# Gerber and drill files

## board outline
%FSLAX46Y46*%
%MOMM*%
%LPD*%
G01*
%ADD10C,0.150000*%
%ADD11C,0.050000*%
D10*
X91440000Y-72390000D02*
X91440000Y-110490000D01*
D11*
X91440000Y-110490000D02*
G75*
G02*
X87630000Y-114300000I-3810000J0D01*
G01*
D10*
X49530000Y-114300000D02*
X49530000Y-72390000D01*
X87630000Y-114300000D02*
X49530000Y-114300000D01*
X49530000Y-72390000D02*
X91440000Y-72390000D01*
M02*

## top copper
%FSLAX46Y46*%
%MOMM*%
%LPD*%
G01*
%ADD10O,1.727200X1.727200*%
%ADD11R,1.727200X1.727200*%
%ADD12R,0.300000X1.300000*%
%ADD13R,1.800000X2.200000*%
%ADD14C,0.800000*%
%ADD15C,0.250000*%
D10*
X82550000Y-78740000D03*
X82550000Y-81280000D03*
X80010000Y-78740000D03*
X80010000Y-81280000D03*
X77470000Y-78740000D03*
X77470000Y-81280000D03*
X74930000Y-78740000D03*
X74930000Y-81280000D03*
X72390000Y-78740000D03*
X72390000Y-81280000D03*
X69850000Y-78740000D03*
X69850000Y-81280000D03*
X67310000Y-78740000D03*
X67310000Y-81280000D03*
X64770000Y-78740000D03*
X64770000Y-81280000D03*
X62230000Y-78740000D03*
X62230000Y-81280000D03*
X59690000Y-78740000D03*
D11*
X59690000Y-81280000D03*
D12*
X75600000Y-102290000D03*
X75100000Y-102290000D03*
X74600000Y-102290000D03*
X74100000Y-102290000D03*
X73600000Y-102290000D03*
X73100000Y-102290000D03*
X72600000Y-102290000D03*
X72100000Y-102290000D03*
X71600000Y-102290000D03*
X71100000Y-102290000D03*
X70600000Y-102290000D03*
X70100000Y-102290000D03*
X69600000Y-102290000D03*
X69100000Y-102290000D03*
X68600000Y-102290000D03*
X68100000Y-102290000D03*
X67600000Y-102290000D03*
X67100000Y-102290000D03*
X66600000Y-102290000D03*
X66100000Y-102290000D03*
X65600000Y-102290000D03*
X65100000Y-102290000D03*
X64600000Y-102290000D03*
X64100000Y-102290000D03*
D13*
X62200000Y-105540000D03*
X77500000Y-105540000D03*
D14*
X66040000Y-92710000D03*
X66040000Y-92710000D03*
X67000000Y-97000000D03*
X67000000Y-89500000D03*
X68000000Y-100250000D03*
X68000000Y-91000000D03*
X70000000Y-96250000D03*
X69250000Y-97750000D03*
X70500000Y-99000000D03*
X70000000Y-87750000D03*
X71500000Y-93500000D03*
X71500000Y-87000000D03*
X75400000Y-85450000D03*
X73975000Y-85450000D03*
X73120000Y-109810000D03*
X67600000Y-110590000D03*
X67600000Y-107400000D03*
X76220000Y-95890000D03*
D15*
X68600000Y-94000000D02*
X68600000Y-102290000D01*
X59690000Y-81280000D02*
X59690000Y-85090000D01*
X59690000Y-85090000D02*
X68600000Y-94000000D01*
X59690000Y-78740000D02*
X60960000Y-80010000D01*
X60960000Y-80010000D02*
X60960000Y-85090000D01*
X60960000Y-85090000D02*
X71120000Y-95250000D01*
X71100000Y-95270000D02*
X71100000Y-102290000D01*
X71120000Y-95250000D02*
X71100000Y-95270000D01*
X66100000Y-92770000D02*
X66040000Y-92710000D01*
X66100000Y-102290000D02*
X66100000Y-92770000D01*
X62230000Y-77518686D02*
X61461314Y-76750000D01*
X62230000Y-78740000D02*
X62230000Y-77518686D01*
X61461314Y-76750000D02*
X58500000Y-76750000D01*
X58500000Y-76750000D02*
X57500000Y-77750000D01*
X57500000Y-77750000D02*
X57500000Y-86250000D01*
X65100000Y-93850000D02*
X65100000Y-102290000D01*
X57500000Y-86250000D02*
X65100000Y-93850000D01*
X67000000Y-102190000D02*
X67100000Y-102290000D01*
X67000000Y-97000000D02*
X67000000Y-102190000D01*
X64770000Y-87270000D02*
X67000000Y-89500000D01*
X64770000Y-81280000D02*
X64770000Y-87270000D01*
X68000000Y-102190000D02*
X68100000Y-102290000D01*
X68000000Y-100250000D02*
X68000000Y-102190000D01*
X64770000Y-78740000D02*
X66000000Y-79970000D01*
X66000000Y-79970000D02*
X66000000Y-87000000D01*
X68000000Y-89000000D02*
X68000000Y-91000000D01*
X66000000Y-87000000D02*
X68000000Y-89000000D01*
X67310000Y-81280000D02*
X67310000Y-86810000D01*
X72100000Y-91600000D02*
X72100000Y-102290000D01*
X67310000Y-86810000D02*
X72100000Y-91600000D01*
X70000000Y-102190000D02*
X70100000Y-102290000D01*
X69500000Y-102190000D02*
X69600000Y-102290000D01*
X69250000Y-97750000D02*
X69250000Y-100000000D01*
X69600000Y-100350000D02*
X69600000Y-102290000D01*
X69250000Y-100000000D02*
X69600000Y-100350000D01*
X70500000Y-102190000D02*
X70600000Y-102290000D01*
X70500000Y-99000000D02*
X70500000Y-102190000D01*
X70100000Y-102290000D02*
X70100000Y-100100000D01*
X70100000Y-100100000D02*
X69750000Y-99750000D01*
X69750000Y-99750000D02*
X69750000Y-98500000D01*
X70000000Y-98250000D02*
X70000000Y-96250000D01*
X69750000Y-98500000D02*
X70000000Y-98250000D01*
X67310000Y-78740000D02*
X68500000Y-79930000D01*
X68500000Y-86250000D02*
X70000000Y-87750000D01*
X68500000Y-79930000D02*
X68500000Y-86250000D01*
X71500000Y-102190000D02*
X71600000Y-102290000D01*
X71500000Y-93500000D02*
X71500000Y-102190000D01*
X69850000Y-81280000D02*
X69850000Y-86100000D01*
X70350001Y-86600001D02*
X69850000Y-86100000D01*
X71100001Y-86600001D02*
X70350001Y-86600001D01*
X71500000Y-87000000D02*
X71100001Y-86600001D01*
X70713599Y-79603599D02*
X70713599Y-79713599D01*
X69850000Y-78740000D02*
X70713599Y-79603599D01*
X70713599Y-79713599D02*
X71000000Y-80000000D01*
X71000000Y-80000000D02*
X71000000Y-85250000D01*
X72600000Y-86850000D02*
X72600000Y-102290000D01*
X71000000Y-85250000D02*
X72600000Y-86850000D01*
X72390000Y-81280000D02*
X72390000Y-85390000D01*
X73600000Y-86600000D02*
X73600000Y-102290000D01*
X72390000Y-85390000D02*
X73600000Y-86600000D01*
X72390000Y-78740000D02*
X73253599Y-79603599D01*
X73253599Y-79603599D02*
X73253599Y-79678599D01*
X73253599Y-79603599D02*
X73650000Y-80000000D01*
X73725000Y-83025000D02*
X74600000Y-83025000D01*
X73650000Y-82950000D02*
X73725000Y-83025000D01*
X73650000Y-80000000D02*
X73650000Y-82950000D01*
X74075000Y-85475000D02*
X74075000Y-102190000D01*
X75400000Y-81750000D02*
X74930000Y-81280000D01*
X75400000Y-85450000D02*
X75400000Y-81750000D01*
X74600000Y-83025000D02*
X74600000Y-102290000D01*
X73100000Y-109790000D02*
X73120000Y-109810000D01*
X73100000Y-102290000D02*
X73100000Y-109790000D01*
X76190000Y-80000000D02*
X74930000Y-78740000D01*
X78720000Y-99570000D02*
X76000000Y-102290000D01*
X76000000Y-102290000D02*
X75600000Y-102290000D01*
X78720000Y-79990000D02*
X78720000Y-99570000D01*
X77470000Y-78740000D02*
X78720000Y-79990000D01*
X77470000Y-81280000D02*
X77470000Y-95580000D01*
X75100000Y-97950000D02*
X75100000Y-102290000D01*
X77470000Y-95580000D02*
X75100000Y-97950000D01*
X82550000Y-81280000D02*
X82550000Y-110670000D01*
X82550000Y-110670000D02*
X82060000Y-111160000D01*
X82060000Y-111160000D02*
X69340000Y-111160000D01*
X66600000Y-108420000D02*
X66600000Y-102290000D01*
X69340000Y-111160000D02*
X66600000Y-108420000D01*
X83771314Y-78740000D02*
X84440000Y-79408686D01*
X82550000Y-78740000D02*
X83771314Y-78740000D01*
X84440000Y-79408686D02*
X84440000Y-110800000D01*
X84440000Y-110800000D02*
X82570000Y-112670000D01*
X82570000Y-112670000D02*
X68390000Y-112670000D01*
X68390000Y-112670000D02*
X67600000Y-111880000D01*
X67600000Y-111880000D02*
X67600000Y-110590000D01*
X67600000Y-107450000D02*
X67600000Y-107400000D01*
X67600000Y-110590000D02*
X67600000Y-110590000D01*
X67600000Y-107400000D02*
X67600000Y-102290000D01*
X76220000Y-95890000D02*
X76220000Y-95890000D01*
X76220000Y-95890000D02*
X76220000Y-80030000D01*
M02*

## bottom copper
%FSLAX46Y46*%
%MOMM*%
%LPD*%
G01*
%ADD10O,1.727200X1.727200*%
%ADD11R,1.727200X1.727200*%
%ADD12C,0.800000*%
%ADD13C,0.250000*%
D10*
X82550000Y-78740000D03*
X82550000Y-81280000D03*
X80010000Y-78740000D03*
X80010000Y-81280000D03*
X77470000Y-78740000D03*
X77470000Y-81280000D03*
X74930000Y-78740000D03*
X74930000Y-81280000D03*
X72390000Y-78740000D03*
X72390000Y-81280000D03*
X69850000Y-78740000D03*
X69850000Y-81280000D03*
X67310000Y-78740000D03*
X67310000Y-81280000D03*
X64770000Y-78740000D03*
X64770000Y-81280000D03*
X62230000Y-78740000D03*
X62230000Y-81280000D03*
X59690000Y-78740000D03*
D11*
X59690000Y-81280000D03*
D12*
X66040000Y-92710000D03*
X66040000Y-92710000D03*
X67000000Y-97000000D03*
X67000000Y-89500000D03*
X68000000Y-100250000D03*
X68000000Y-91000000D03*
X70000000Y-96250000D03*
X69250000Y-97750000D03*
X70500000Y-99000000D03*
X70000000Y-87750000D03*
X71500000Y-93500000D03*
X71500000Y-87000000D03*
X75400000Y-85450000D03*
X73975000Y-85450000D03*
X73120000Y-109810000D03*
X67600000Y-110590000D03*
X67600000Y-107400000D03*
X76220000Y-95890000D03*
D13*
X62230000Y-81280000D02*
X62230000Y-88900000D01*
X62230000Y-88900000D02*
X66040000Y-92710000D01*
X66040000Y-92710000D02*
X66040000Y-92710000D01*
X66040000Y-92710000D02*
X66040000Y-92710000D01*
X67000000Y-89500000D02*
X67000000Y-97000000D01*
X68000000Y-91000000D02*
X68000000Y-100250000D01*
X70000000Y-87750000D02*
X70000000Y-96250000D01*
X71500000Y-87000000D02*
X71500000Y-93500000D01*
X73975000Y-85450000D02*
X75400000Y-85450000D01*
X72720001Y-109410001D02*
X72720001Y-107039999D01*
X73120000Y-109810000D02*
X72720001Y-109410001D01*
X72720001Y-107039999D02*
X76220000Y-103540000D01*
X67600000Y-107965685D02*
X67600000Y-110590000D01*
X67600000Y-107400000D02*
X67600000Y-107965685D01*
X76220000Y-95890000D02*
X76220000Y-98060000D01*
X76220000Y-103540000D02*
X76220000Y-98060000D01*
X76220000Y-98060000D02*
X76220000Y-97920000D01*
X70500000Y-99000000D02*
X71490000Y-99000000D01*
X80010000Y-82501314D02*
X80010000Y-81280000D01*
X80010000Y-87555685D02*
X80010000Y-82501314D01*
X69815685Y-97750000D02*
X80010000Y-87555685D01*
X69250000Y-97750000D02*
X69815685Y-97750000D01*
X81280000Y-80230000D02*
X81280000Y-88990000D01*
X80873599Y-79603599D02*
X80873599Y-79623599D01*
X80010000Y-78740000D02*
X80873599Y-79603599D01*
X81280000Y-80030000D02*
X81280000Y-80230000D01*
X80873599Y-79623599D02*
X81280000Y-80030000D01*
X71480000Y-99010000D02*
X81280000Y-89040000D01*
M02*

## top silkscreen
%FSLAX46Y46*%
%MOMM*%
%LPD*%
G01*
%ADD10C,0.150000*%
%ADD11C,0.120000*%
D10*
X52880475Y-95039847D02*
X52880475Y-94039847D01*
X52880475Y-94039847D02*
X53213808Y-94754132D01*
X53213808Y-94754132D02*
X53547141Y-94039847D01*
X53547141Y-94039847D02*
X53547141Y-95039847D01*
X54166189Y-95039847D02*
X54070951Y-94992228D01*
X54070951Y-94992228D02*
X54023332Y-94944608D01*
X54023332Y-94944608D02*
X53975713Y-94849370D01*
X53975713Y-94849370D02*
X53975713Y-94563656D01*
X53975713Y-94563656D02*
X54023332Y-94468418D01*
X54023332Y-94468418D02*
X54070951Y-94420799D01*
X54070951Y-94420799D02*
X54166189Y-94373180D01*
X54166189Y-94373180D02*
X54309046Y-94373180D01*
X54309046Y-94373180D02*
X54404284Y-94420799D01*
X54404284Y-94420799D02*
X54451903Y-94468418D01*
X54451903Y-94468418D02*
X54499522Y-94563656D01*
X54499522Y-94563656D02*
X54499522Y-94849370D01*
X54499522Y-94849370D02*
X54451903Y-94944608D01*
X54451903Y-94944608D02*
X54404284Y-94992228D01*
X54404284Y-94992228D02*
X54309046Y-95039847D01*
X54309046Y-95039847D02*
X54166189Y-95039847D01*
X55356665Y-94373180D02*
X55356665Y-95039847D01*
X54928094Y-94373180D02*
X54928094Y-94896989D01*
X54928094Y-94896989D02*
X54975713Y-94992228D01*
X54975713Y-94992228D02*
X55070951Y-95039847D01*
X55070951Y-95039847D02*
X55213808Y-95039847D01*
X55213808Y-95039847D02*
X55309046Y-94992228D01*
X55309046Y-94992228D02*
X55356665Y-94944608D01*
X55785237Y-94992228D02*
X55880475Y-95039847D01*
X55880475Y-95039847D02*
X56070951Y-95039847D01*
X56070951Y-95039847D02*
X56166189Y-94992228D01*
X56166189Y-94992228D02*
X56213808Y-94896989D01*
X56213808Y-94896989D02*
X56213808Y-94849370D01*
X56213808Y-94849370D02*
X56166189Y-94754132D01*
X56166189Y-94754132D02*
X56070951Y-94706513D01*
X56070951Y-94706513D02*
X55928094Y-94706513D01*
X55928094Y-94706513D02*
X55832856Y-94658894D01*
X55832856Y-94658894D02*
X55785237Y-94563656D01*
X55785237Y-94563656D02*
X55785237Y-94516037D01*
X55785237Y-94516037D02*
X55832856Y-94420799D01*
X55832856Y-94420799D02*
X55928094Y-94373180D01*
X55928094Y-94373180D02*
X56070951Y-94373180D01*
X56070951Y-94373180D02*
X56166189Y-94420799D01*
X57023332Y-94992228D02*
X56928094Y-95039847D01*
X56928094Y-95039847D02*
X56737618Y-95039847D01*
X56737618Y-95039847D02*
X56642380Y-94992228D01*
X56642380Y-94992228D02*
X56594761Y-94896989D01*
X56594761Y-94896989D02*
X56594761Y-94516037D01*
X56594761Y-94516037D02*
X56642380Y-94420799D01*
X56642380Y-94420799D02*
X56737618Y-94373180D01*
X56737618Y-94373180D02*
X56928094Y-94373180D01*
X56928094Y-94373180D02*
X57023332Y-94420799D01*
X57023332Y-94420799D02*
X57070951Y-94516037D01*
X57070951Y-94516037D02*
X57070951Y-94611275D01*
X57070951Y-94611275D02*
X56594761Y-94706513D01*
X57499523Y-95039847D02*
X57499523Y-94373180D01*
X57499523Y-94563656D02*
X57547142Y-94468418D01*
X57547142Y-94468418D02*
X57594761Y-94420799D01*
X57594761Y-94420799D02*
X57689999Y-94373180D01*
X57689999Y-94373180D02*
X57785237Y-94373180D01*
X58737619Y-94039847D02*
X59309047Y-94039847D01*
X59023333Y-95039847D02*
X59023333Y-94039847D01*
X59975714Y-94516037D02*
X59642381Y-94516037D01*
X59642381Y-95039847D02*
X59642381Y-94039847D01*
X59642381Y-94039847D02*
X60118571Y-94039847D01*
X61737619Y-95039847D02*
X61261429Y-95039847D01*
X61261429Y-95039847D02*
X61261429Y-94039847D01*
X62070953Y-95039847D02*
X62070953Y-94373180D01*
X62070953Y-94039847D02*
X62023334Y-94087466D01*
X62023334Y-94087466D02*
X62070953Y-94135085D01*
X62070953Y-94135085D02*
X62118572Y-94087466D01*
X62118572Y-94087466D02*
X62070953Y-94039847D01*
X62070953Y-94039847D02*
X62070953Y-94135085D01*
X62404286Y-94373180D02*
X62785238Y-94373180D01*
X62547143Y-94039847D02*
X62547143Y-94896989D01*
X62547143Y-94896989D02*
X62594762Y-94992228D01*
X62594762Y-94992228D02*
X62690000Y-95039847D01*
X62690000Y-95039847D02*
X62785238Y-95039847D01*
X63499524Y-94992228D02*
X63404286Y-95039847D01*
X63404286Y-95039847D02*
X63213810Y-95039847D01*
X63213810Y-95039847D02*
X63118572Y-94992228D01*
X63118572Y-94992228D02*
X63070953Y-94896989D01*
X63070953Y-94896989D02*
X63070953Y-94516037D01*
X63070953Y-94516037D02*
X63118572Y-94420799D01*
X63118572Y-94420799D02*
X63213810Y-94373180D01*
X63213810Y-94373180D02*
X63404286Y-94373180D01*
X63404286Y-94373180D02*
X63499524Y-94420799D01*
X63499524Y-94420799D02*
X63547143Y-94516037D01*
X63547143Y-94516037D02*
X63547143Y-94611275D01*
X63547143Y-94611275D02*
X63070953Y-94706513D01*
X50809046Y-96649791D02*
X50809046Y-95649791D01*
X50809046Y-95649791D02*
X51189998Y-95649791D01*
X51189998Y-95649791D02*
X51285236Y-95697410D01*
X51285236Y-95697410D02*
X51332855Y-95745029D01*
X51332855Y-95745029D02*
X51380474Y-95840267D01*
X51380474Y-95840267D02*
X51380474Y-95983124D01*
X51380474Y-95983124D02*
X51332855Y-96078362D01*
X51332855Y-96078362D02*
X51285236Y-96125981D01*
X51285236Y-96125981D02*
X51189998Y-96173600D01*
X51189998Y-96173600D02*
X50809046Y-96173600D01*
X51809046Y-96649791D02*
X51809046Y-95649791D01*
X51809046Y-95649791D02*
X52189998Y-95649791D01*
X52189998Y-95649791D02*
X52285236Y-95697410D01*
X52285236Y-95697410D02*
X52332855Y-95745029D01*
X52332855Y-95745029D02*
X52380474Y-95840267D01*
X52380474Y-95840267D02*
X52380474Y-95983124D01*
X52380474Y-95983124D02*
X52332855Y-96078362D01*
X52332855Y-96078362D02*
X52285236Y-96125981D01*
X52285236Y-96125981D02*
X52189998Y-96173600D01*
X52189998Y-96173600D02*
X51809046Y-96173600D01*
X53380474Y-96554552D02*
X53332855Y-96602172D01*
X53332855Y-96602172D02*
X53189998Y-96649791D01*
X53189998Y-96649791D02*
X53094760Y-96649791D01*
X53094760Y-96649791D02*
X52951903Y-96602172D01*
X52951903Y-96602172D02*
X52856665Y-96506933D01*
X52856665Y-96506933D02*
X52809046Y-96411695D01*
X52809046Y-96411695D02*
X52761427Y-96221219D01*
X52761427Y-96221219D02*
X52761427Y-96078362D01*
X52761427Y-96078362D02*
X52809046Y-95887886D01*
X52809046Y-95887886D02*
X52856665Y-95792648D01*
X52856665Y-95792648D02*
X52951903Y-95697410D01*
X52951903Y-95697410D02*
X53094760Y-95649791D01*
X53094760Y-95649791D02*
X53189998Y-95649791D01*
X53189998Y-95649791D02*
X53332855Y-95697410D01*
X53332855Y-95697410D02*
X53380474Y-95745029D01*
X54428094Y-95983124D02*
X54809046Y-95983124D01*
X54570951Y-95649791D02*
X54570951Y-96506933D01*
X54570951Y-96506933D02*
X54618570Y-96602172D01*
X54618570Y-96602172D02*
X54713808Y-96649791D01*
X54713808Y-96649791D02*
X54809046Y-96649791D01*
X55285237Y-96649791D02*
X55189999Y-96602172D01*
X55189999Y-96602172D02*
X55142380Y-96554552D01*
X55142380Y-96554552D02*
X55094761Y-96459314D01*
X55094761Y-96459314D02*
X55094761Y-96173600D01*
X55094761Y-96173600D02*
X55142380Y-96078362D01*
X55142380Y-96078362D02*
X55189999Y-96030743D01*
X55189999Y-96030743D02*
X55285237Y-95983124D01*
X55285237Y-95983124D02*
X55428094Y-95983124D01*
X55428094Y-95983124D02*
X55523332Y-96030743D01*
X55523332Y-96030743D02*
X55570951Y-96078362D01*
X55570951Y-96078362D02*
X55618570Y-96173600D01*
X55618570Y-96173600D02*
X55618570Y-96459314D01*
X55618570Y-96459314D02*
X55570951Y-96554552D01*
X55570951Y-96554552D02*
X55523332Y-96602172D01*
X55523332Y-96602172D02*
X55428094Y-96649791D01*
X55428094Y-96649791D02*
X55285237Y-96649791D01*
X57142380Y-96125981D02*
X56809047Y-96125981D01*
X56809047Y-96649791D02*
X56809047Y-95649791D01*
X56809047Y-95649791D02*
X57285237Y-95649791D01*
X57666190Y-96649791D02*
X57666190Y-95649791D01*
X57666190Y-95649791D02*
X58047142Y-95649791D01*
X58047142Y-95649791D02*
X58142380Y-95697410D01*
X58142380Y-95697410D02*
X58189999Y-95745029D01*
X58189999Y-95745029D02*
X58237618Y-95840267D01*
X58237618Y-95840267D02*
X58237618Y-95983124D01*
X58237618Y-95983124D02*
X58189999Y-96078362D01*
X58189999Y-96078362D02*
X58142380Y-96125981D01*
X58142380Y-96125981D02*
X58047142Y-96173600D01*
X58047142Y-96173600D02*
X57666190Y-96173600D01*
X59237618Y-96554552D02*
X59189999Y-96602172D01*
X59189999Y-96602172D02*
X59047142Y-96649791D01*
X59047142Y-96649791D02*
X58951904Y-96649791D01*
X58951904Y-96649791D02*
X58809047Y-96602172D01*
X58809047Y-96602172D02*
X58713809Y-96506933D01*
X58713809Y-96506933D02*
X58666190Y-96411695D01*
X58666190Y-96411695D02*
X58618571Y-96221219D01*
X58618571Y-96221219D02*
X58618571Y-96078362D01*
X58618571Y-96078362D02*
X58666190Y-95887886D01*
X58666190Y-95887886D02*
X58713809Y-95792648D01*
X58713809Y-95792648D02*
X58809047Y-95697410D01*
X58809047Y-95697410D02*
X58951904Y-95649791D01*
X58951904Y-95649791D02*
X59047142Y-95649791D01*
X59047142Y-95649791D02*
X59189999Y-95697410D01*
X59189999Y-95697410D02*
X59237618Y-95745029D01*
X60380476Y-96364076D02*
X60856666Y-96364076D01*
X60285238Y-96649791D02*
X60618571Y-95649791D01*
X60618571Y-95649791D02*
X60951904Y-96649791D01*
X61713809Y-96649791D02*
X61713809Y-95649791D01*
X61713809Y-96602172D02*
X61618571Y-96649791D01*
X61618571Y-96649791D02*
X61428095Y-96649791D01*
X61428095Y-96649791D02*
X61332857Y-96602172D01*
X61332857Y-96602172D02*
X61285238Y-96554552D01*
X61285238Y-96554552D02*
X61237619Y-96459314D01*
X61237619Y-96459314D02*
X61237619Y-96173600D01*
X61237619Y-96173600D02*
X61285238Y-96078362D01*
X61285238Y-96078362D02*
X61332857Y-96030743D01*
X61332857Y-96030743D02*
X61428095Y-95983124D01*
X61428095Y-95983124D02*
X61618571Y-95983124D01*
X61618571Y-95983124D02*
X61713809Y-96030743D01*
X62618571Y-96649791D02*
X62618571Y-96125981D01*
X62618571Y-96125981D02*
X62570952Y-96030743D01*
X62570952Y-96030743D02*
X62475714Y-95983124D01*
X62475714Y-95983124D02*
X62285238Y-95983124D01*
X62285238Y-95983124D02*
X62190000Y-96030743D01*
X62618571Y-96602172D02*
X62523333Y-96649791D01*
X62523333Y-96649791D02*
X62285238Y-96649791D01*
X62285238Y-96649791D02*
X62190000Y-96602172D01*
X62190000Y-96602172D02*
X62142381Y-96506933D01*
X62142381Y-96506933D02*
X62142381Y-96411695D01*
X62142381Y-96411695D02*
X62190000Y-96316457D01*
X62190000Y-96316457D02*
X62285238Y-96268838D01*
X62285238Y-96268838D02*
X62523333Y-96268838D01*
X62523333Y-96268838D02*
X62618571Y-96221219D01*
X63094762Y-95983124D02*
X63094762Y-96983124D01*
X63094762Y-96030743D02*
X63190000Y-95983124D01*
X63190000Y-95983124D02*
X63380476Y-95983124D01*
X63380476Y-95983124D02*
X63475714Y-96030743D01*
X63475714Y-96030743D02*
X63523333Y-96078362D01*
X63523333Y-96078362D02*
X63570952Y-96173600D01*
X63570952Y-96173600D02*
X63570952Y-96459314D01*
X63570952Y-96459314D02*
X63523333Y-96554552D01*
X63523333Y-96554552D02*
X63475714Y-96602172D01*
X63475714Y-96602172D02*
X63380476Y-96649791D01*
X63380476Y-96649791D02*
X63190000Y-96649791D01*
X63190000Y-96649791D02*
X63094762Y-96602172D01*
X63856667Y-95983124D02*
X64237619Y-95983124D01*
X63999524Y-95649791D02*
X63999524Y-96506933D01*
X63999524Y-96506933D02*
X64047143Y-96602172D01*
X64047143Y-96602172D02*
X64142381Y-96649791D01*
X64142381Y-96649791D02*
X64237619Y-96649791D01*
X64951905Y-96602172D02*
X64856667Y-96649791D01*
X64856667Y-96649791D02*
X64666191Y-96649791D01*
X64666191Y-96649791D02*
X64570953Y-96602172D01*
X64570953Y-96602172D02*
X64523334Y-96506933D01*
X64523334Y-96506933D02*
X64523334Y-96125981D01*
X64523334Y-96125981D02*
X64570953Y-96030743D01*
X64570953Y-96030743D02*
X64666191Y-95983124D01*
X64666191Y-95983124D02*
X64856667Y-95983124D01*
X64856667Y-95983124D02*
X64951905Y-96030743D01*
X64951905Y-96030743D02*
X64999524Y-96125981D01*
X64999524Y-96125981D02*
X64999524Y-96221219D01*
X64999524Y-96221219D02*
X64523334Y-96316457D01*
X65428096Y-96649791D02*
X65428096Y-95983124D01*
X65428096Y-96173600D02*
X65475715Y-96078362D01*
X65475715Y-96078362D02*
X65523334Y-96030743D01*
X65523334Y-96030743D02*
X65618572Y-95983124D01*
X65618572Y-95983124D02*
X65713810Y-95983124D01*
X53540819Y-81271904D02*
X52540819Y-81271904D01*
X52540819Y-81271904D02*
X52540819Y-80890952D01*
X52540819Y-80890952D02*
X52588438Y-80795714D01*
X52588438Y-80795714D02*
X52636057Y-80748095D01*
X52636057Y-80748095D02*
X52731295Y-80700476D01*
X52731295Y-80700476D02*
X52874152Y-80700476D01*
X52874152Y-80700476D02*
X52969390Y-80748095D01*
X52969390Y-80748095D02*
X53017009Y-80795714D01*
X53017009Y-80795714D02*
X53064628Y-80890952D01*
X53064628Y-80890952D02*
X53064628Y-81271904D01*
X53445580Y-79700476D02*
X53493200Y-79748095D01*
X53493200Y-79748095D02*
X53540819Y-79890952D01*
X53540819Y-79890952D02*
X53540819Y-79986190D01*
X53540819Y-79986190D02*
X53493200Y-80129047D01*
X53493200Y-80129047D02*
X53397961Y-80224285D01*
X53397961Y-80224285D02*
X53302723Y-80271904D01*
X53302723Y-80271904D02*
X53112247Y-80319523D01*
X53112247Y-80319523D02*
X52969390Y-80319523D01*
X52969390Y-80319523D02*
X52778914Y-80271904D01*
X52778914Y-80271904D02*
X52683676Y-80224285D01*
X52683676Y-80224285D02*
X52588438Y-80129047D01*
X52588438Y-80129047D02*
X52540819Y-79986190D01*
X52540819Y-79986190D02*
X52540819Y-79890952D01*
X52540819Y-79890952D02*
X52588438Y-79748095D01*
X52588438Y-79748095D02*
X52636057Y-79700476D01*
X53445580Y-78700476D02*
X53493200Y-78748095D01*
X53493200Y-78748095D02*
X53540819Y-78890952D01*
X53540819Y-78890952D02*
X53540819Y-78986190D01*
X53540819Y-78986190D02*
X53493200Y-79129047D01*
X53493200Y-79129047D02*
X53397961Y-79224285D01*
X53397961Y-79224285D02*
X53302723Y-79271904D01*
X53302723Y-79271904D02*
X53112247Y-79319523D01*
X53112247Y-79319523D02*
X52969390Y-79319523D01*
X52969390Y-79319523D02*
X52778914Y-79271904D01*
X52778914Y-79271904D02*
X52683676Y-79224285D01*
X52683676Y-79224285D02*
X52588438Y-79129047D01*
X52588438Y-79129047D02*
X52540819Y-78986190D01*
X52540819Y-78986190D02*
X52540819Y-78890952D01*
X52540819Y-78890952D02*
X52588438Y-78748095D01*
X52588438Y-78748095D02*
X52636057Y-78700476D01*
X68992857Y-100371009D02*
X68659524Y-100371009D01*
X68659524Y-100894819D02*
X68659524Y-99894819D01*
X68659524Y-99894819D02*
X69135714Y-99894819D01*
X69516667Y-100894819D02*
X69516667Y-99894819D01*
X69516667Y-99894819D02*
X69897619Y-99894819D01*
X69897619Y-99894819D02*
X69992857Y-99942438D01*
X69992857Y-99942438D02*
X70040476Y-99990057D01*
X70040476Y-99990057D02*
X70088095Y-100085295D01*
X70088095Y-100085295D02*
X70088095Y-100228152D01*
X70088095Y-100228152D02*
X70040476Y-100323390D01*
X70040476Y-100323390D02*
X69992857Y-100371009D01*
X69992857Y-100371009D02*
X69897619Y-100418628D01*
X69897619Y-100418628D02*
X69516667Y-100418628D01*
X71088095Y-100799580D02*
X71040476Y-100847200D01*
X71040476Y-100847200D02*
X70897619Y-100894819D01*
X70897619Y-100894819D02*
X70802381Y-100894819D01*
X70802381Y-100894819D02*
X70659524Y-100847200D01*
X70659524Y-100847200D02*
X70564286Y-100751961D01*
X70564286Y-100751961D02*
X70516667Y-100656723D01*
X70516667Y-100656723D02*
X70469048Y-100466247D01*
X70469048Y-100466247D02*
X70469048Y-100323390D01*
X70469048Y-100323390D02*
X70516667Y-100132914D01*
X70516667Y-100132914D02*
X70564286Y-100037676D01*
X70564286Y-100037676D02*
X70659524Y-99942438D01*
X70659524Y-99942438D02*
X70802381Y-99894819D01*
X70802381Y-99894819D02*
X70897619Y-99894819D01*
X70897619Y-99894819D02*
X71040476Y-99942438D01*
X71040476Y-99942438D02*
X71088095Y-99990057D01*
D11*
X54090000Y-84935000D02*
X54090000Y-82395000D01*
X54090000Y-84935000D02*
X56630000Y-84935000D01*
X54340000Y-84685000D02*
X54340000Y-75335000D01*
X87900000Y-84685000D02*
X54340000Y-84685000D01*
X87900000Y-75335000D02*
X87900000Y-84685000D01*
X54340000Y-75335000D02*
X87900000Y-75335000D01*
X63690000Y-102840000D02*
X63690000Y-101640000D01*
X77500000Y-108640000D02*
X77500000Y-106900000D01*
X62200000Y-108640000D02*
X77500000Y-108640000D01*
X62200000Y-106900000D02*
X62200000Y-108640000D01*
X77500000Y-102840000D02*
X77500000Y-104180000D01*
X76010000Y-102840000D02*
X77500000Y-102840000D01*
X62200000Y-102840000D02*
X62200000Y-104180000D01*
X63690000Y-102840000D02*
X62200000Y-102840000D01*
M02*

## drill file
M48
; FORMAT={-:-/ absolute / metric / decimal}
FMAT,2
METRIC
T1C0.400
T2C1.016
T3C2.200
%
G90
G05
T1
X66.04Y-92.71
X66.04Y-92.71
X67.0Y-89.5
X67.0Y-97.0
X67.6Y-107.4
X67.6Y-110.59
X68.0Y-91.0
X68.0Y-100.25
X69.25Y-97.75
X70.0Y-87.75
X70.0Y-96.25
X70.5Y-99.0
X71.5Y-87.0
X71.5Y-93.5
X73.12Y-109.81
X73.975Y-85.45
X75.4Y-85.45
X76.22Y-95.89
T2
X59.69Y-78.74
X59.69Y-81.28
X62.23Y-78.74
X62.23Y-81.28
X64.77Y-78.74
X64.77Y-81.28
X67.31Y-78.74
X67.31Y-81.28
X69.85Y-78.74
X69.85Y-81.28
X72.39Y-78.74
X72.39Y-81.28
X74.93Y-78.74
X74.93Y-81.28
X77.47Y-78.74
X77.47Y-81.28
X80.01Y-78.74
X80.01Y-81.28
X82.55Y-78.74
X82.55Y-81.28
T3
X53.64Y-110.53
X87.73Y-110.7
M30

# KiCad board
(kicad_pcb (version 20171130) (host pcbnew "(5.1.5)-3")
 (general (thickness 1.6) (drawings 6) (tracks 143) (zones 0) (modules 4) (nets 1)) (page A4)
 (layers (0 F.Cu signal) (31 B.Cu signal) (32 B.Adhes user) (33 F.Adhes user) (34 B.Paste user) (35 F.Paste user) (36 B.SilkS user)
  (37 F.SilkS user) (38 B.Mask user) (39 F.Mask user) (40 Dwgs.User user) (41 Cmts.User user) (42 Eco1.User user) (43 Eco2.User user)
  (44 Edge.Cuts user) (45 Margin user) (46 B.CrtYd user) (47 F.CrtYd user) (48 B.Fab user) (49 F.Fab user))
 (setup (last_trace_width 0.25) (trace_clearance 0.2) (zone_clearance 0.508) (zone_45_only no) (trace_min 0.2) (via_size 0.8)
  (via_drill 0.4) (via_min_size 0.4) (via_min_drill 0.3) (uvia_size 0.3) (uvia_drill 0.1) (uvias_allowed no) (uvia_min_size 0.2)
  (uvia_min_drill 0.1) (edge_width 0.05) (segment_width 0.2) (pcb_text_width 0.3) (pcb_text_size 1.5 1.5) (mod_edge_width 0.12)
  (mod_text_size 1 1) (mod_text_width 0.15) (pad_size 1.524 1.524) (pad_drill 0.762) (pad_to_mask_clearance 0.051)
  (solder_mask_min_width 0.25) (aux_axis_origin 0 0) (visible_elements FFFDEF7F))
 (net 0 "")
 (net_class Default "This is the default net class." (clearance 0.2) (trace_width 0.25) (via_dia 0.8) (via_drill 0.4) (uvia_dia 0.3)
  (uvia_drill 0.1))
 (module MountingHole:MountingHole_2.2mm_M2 (layer F.Cu) (at 87.73 110.7)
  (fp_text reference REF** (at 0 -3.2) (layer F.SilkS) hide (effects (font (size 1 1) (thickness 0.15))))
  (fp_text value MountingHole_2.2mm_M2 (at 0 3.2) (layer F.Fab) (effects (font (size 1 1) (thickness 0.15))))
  (pad 1 np_thru_hole circle (at 0 0) (size 2.2 2.2) (drill 2.2) (layers *.Cu *.Mask)))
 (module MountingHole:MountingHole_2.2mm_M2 (layer F.Cu) (at 53.64 110.53)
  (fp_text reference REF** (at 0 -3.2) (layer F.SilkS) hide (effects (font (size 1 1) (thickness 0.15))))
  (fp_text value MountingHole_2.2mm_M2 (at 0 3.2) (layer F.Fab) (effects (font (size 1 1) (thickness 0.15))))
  (pad 1 np_thru_hole circle (at 0 0) (size 2.2 2.2) (drill 2.2) (layers *.Cu *.Mask)))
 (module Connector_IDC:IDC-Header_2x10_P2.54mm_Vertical (layer F.Cu) (at 59.69 81.28 90)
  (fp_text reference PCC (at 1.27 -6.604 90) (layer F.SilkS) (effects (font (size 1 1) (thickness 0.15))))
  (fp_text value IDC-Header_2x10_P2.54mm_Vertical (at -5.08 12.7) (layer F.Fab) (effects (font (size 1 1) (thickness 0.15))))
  (fp_line (start -3.655 -5.6) (end -1.115 -5.6) (layer F.SilkS) (width 0.12))
  (fp_line (start -3.655 -5.6) (end -3.655 -3.06) (layer F.SilkS) (width 0.12))
  (fp_line (start -3.405 -5.35) (end 5.945 -5.35) (layer F.SilkS) (width 0.12))
  (fp_line (start -3.405 28.21) (end -3.405 -5.35) (layer F.SilkS) (width 0.12))
  (fp_line (start 5.945 28.21) (end -3.405 28.21) (layer F.SilkS) (width 0.12))
  (fp_line (start 5.945 -5.35) (end 5.945 28.21) (layer F.SilkS) (width 0.12))
  (pad 20 thru_hole oval (at 2.54 22.86 90) (size 1.7272 1.7272) (drill 1.016) (layers *.Cu *.Mask))
  (pad 19 thru_hole oval (at 0 22.86 90) (size 1.7272 1.7272) (drill 1.016) (layers *.Cu *.Mask))
  (pad 18 thru_hole oval (at 2.54 20.32 90) (size 1.7272 1.7272) (drill 1.016) (layers *.Cu *.Mask))
  (pad 17 thru_hole oval (at 0 20.32 90) (size 1.7272 1.7272) (drill 1.016) (layers *.Cu *.Mask))
  (pad 16 thru_hole oval (at 2.54 17.78 90) (size 1.7272 1.7272) (drill 1.016) (layers *.Cu *.Mask))
  (pad 15 thru_hole oval (at 0 17.78 90) (size 1.7272 1.7272) (drill 1.016) (layers *.Cu *.Mask))
  (pad 14 thru_hole oval (at 2.54 15.24 90) (size 1.7272 1.7272) (drill 1.016) (layers *.Cu *.Mask))
  (pad 13 thru_hole oval (at 0 15.24 90) (size 1.7272 1.7272) (drill 1.016) (layers *.Cu *.Mask))
  (pad 12 thru_hole oval (at 2.54 12.7 90) (size 1.7272 1.7272) (drill 1.016) (layers *.Cu *.Mask))
  (pad 11 thru_hole oval (at 0 12.7 90) (size 1.7272 1.7272) (drill 1.016) (layers *.Cu *.Mask))
  (pad 10 thru_hole oval (at 2.54 10.16 90) (size 1.7272 1.7272) (drill 1.016) (layers *.Cu *.Mask))
  (pad 9 thru_hole oval (at 0 10.16 90) (size 1.7272 1.7272) (drill 1.016) (layers *.Cu *.Mask))
  (pad 8 thru_hole oval (at 2.54 7.62 90) (size 1.7272 1.7272) (drill 1.016) (layers *.Cu *.Mask))
  (pad 7 thru_hole oval (at 0 7.62 90) (size 1.7272 1.7272) (drill 1.016) (layers *.Cu *.Mask))
  (pad 6 thru_hole oval (at 2.54 5.08 90) (size 1.7272 1.7272) (drill 1.016) (layers *.Cu *.Mask))
  (pad 5 thru_hole oval (at 0 5.08 90) (size 1.7272 1.7272) (drill 1.016) (layers *.Cu *.Mask))
  (pad 4 thru_hole oval (at 2.54 2.54 90) (size 1.7272 1.7272) (drill 1.016) (layers *.Cu *.Mask))
  (pad 3 thru_hole oval (at 0 2.54 90) (size 1.7272 1.7272) (drill 1.016) (layers *.Cu *.Mask))
  (pad 2 thru_hole oval (at 2.54 0 90) (size 1.7272 1.7272) (drill 1.016) (layers *.Cu *.Mask))
  (pad 1 thru_hole rect (at 0 0 90) (size 1.7272 1.7272) (drill 1.016) (layers *.Cu *.Mask)))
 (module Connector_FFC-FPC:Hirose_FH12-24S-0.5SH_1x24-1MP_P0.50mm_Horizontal (layer F.Cu) (at 69.85 104.14)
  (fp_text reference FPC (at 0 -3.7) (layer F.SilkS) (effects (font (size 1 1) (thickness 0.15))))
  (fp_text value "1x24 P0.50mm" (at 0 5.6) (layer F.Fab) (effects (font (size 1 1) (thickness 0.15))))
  (fp_line (start -6.16 -1.3) (end -6.16 -2.5) (layer F.SilkS) (width 0.12))
  (fp_line (start 7.65 4.5) (end 7.65 2.76) (layer F.SilkS) (width 0.12))
  (fp_line (start -7.65 4.5) (end 7.65 4.5) (layer F.SilkS) (width 0.12))
  (fp_line (start -7.65 2.76) (end -7.65 4.5) (layer F.SilkS) (width 0.12))
  (fp_line (start 7.65 -1.3) (end 7.65 0.04) (layer F.SilkS) (width 0.12))
  (fp_line (start 6.16 -1.3) (end 7.65 -1.3) (layer F.SilkS) (width 0.12))
  (fp_line (start -7.65 -1.3) (end -7.65 0.04) (layer F.SilkS) (width 0.12))
  (fp_line (start -6.16 -1.3) (end -7.65 -1.3) (layer F.SilkS) (width 0.12))
  (pad 24 smd rect (at 5.75 -1.85) (size 0.3 1.3) (layers F.Cu F.Paste F.Mask))
  (pad 23 smd rect (at 5.25 -1.85) (size 0.3 1.3) (layers F.Cu F.Paste F.Mask))
  (pad 22 smd rect (at 4.75 -1.85) (size 0.3 1.3) (layers F.Cu F.Paste F.Mask))
  (pad 21 smd rect (at 4.25 -1.85) (size 0.3 1.3) (layers F.Cu F.Paste F.Mask))
  (pad 20 smd rect (at 3.75 -1.85) (size 0.3 1.3) (layers F.Cu F.Paste F.Mask))
  (pad 19 smd rect (at 3.25 -1.85) (size 0.3 1.3) (layers F.Cu F.Paste F.Mask))
  (pad 18 smd rect (at 2.75 -1.85) (size 0.3 1.3) (layers F.Cu F.Paste F.Mask))
  (pad 17 smd rect (at 2.25 -1.85) (size 0.3 1.3) (layers F.Cu F.Paste F.Mask))
  (pad 16 smd rect (at 1.75 -1.85) (size 0.3 1.3) (layers F.Cu F.Paste F.Mask))
  (pad 15 smd rect (at 1.25 -1.85) (size 0.3 1.3) (layers F.Cu F.Paste F.Mask))
  (pad 14 smd rect (at 0.75 -1.85) (size 0.3 1.3) (layers F.Cu F.Paste F.Mask))
  (pad 13 smd rect (at 0.25 -1.85) (size 0.3 1.3) (layers F.Cu F.Paste F.Mask))
  (pad 12 smd rect (at -0.25 -1.85) (size 0.3 1.3) (layers F.Cu F.Paste F.Mask))
  (pad 11 smd rect (at -0.75 -1.85) (size 0.3 1.3) (layers F.Cu F.Paste F.Mask))
  (pad 10 smd rect (at -1.25 -1.85) (size 0.3 1.3) (layers F.Cu F.Paste F.Mask))
  (pad 9 smd rect (at -1.75 -1.85) (size 0.3 1.3) (layers F.Cu F.Paste F.Mask))
  (pad 8 smd rect (at -2.25 -1.85) (size 0.3 1.3) (layers F.Cu F.Paste F.Mask))
  (pad 7 smd rect (at -2.75 -1.85) (size 0.3 1.3) (layers F.Cu F.Paste F.Mask))
  (pad 6 smd rect (at -3.25 -1.85) (size 0.3 1.3) (layers F.Cu F.Paste F.Mask))
  (pad 5 smd rect (at -3.75 -1.85) (size 0.3 1.3) (layers F.Cu F.Paste F.Mask))
  (pad 4 smd rect (at -4.25 -1.85) (size 0.3 1.3) (layers F.Cu F.Paste F.Mask))
  (pad 3 smd rect (at -4.75 -1.85) (size 0.3 1.3) (layers F.Cu F.Paste F.Mask))
  (pad 2 smd rect (at -5.25 -1.85) (size 0.3 1.3) (layers F.Cu F.Paste F.Mask))
  (pad 1 smd rect (at -5.75 -1.85) (size 0.3 1.3) (layers F.Cu F.Paste F.Mask))
  (pad MP smd rect (at -7.65 1.4) (size 1.8 2.2) (layers F.Cu F.Paste F.Mask))
  (pad MP smd rect (at 7.65 1.4) (size 1.8 2.2) (layers F.Cu F.Paste F.Mask)))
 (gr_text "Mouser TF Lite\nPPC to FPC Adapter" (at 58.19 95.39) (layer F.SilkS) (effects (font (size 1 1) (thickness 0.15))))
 (gr_line (start 91.44 72.39) (end 91.44 110.49) (layer Edge.Cuts) (width 0.15))
 (gr_arc (start 87.63 110.49) (end 87.63 114.3) (angle -90) (layer Edge.Cuts) (width 0.05))
 (gr_line (start 49.53 114.3) (end 49.53 72.39) (layer Edge.Cuts) (width 0.15))
 (gr_line (start 87.63 114.3) (end 49.53 114.3) (layer Edge.Cuts) (width 0.15))
 (gr_line (start 49.53 72.39) (end 91.44 72.39) (layer Edge.Cuts) (width 0.15))
 (segment (start 68.6 94) (end 68.6 102.29) (width 0.25) (layer F.Cu) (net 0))
 (segment (start 59.69 81.28) (end 59.69 85.09) (width 0.25) (layer F.Cu) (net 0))
 (segment (start 59.69 85.09) (end 68.6 94) (width 0.25) (layer F.Cu) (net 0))
 (segment (start 59.69 78.74) (end 60.96 80.01) (width 0.25) (layer F.Cu) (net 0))
 (segment (start 60.96 80.01) (end 60.96 85.09) (width 0.25) (layer F.Cu) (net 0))
 (segment (start 60.96 85.09) (end 71.12 95.25) (width 0.25) (layer F.Cu) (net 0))
 (segment (start 71.1 95.27) (end 71.1 102.29) (width 0.25) (layer F.Cu) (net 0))
 (segment (start 71.12 95.25) (end 71.1 95.27) (width 0.25) (layer F.Cu) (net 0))
 (segment (start 62.23 81.28) (end 62.23 88.9) (width 0.25) (layer B.Cu) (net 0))
 (segment (start 62.23 88.9) (end 66.04 92.71) (width 0.25) (layer B.Cu) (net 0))
 (segment (start 66.04 92.71) (end 66.04 92.71) (width 0.25) (layer B.Cu) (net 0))
 (via (at 66.04 92.71) (size 0.8) (drill 0.4) (layers F.Cu B.Cu) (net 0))
 (segment (start 66.04 92.71) (end 66.04 92.71) (width 0.25) (layer B.Cu) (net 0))
 (via (at 66.04 92.71) (size 0.8) (drill 0.4) (layers F.Cu B.Cu) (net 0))
 (segment (start 66.1 92.77) (end 66.04 92.71) (width 0.25) (layer F.Cu) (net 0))
 (segment (start 66.1 102.29) (end 66.1 92.77) (width 0.25) (layer F.Cu) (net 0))
 (segment (start 62.23 77.518686) (end 61.461314 76.75) (width 0.25) (layer F.Cu) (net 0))
 (segment (start 62.23 78.74) (end 62.23 77.518686) (width 0.25) (layer F.Cu) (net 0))
 (segment (start 61.461314 76.75) (end 58.5 76.75) (width 0.25) (layer F.Cu) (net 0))
 (segment (start 58.5 76.75) (end 57.5 77.75) (width 0.25) (layer F.Cu) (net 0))
 (segment (start 57.5 77.75) (end 57.5 86.25) (width 0.25) (layer F.Cu) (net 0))
 (segment (start 65.1 93.85) (end 65.1 102.29) (width 0.25) (layer F.Cu) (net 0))
 (segment (start 57.5 86.25) (end 65.1 93.85) (width 0.25) (layer F.Cu) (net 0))
 (via (at 67 97) (size 0.8) (drill 0.4) (layers F.Cu B.Cu) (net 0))
 (segment (start 67 102.19) (end 67.1 102.29) (width 0.25) (layer F.Cu) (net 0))
 (segment (start 67 97) (end 67 102.19) (width 0.25) (layer F.Cu) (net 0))
 (via (at 67 89.5) (size 0.8) (drill 0.4) (layers F.Cu B.Cu) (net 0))
 (segment (start 67 89.5) (end 67 97) (width 0.25) (layer B.Cu) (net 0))
 (segment (start 64.77 87.27) (end 67 89.5) (width 0.25) (layer F.Cu) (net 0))
 (segment (start 64.77 81.28) (end 64.77 87.27) (width 0.25) (layer F.Cu) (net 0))
 (via (at 68 100.25) (size 0.8) (drill 0.4) (layers F.Cu B.Cu) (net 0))
 (segment (start 68 102.19) (end 68.1 102.29) (width 0.25) (layer F.Cu) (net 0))
 (segment (start 68 100.25) (end 68 102.19) (width 0.25) (layer F.Cu) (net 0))
 (via (at 68 91) (size 0.8) (drill 0.4) (layers F.Cu B.Cu) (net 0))
 (segment (start 64.77 78.74) (end 66 79.97) (width 0.25) (layer F.Cu) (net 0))
 (segment (start 66 79.97) (end 66 87) (width 0.25) (layer F.Cu) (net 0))
 (segment (start 68 89) (end 68 91) (width 0.25) (layer F.Cu) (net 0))
 (segment (start 66 87) (end 68 89) (width 0.25) (layer F.Cu) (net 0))
 (segment (start 68 91) (end 68 100.25) (width 0.25) (layer B.Cu) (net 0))
 (segment (start 67.31 81.28) (end 67.31 86.81) (width 0.25) (layer F.Cu) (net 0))
 (segment (start 72.1 91.6) (end 72.1 102.29) (width 0.25) (layer F.Cu) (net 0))
 (segment (start 67.31 86.81) (end 72.1 91.6) (width 0.25) (layer F.Cu) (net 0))
 (via (at 70 96.25) (size 0.8) (drill 0.4) (layers F.Cu B.Cu) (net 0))
 (via (at 69.25 97.75) (size 0.8) (drill 0.4) (layers F.Cu B.Cu) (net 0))
 (segment (start 70 102.19) (end 70.1 102.29) (width 0.25) (layer F.Cu) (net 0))
 (segment (start 69.5 102.19) (end 69.6 102.29) (width 0.25) (layer F.Cu) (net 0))
 (segment (start 69.25 97.75) (end 69.25 100) (width 0.25) (layer F.Cu) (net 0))
 (segment (start 69.6 100.35) (end 69.6 102.29) (width 0.25) (layer F.Cu) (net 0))
 (segment (start 69.25 100) (end 69.6 100.35) (width 0.25) (layer F.Cu) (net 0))
 (via (at 70.5 99) (size 0.8) (drill 0.4) (layers F.Cu B.Cu) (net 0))
 (segment (start 70.5 102.19) (end 70.6 102.29) (width 0.25) (layer F.Cu) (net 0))
 (segment (start 70.5 99) (end 70.5 102.19) (width 0.25) (layer F.Cu) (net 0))
 (segment (start 70.1 102.29) (end 70.1 100.1) (width 0.25) (layer F.Cu) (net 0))
 (segment (start 70.1 100.1) (end 69.75 99.75) (width 0.25) (layer F.Cu) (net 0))
 (segment (start 69.75 99.75) (end 69.75 98.5) (width 0.25) (layer F.Cu) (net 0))
 (segment (start 70 98.25) (end 70 96.25) (width 0.25) (layer F.Cu) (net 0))
 (segment (start 69.75 98.5) (end 70 98.25) (width 0.25) (layer F.Cu) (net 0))
 (via (at 70 87.75) (size 0.8) (drill 0.4) (layers F.Cu B.Cu) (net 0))
 (segment (start 67.31 78.74) (end 68.5 79.93) (width 0.25) (layer F.Cu) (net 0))
 (segment (start 68.5 86.25) (end 70 87.75) (width 0.25) (layer F.Cu) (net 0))
 (segment (start 68.5 79.93) (end 68.5 86.25) (width 0.25) (layer F.Cu) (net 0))
 (segment (start 70 87.75) (end 70 96.25) (width 0.25) (layer B.Cu) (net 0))
 (via (at 71.5 93.5) (size 0.8) (drill 0.4) (layers F.Cu B.Cu) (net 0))
 (segment (start 71.5 102.19) (end 71.6 102.29) (width 0.25) (layer F.Cu) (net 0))
 (segment (start 71.5 93.5) (end 71.5 102.19) (width 0.25) (layer F.Cu) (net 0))
 (segment (start 69.85 81.28) (end 69.85 86.1) (width 0.25) (layer F.Cu) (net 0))
 (via (at 71.5 87) (size 0.8) (drill 0.4) (layers F.Cu B.Cu) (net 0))
 (segment (start 70.350001 86.600001) (end 69.85 86.1) (width 0.25) (layer F.Cu) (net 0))
 (segment (start 71.100001 86.600001) (end 70.350001 86.600001) (width 0.25) (layer F.Cu) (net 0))
 (segment (start 71.5 87) (end 71.100001 86.600001) (width 0.25) (layer F.Cu) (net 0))
 (segment (start 71.5 87) (end 71.5 93.5) (width 0.25) (layer B.Cu) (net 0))
 (segment (start 70.713599 79.603599) (end 70.713599 79.713599) (width 0.25) (layer F.Cu) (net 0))
 (segment (start 69.85 78.74) (end 70.713599 79.603599) (width 0.25) (layer F.Cu) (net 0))
 (segment (start 70.713599 79.713599) (end 71 80) (width 0.25) (layer F.Cu) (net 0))
 (segment (start 71 80) (end 71 85.25) (width 0.25) (layer F.Cu) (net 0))
 (segment (start 72.6 86.85) (end 72.6 102.29) (width 0.25) (layer F.Cu) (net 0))
 (segment (start 71 85.25) (end 72.6 86.85) (width 0.25) (layer F.Cu) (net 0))
 (segment (start 72.39 81.28) (end 72.39 85.39) (width 0.25) (layer F.Cu) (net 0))
 (segment (start 73.6 86.6) (end 73.6 102.29) (width 0.25) (layer F.Cu) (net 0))
 (segment (start 72.39 85.39) (end 73.6 86.6) (width 0.25) (layer F.Cu) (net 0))
 (segment (start 72.39 78.74) (end 73.253599 79.603599) (width 0.25) (layer F.Cu) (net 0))
 (segment (start 73.253599 79.603599) (end 73.253599 79.678599) (width 0.25) (layer F.Cu) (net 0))
 (segment (start 73.253599 79.603599) (end 73.65 80) (width 0.25) (layer F.Cu) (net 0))
 (segment (start 73.725 83.025) (end 74.6 83.025) (width 0.25) (layer F.Cu) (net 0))
 (segment (start 73.65 82.95) (end 73.725 83.025) (width 0.25) (layer F.Cu) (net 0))
 (segment (start 73.65 80) (end 73.65 82.95) (width 0.25) (layer F.Cu) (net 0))
 (via (at 75.4 85.45) (size 0.8) (drill 0.4) (layers F.Cu B.Cu) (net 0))
 (via (at 73.975 85.45) (size 0.8) (drill 0.4) (layers F.Cu B.Cu) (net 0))
 (segment (start 74.075 85.475) (end 74.075 102.19) (width 0.25) (layer F.Cu) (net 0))
 (segment (start 73.975 85.45) (end 75.4 85.45) (width 0.25) (layer B.Cu) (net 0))
 (segment (start 75.4 81.75) (end 74.93 81.28) (width 0.25) (layer F.Cu) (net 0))
 (segment (start 75.4 85.45) (end 75.4 81.75) (width 0.25) (layer F.Cu) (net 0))
 (segment (start 74.6 83.025) (end 74.6 102.29) (width 0.25) (layer F.Cu) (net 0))
 (via (at 73.12 109.81) (size 0.8) (drill 0.4) (layers F.Cu B.Cu) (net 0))
 (segment (start 73.1 109.79) (end 73.12 109.81) (width 0.25) (layer F.Cu) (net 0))
 (segment (start 73.1 102.29) (end 73.1 109.79) (width 0.25) (layer F.Cu) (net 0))
 (segment (start 76.19 80) (end 74.93 78.74) (width 0.25) (layer F.Cu) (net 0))
 (segment (start 72.720001 109.410001) (end 72.720001 107.039999) (width 0.25) (layer B.Cu) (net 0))
 (segment (start 73.12 109.81) (end 72.720001 109.410001) (width 0.25) (layer B.Cu) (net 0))
 (segment (start 72.720001 107.039999) (end 76.22 103.54) (width 0.25) (layer B.Cu) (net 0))
 (segment (start 78.72 99.57) (end 76 102.29) (width 0.25) (layer F.Cu) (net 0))
 (segment (start 76 102.29) (end 75.6 102.29) (width 0.25) (layer F.Cu) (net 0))
 (segment (start 78.72 79.99) (end 78.72 99.57) (width 0.25) (layer F.Cu) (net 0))
 (segment (start 77.47 78.74) (end 78.72 79.99) (width 0.25) (layer F.Cu) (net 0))
 (segment (start 77.47 81.28) (end 77.47 95.58) (width 0.25) (layer F.Cu) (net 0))
 (segment (start 75.1 97.95) (end 75.1 102.29) (width 0.25) (layer F.Cu) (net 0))
 (segment (start 77.47 95.58) (end 75.1 97.95) (width 0.25) (layer F.Cu) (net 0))
 (segment (start 82.55 81.28) (end 82.55 110.67) (width 0.25) (layer F.Cu) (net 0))
 (segment (start 82.55 110.67) (end 82.06 111.16) (width 0.25) (layer F.Cu) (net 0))
 (segment (start 82.06 111.16) (end 69.34 111.16) (width 0.25) (layer F.Cu) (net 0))
 (segment (start 66.6 108.42) (end 66.6 102.29) (width 0.25) (layer F.Cu) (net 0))
 (segment (start 69.34 111.16) (end 66.6 108.42) (width 0.25) (layer F.Cu) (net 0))
 (segment (start 83.771314 78.74) (end 84.44 79.408686) (width 0.25) (layer F.Cu) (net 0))
 (segment (start 82.55 78.74) (end 83.771314 78.74) (width 0.25) (layer F.Cu) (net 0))
 (segment (start 84.44 79.408686) (end 84.44 110.8) (width 0.25) (layer F.Cu) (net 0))
 (segment (start 84.44 110.8) (end 82.57 112.67) (width 0.25) (layer F.Cu) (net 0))
 (segment (start 82.57 112.67) (end 68.39 112.67) (width 0.25) (layer F.Cu) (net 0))
 (segment (start 68.39 112.67) (end 67.6 111.88) (width 0.25) (layer F.Cu) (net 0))
 (segment (start 67.6 111.88) (end 67.6 110.59) (width 0.25) (layer F.Cu) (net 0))
 (segment (start 67.6 107.45) (end 67.6 107.4) (width 0.25) (layer F.Cu) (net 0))
 (segment (start 67.6 110.59) (end 67.6 110.59) (width 0.25) (layer F.Cu) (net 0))
 (via (at 67.6 110.59) (size 0.8) (drill 0.4) (layers F.Cu B.Cu) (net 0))
 (segment (start 67.6 107.4) (end 67.6 102.29) (width 0.25) (layer F.Cu) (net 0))
 (via (at 67.6 107.4) (size 0.8) (drill 0.4) (layers F.Cu B.Cu) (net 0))
 (segment (start 67.6 107.965685) (end 67.6 110.59) (width 0.25) (layer B.Cu) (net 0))
 (segment (start 67.6 107.4) (end 67.6 107.965685) (width 0.25) (layer B.Cu) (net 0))
 (segment (start 76.22 95.89) (end 76.22 95.89) (width 0.25) (layer F.Cu) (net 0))
 (segment (start 76.22 95.89) (end 76.22 80.03) (width 0.25) (layer F.Cu) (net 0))
 (via (at 76.22 95.89) (size 0.8) (drill 0.4) (layers F.Cu B.Cu) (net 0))
 (segment (start 76.22 95.89) (end 76.22 98.06) (width 0.25) (layer B.Cu) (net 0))
 (segment (start 76.22 103.54) (end 76.22 98.06) (width 0.25) (layer B.Cu) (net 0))
 (segment (start 76.22 98.06) (end 76.22 97.92) (width 0.25) (layer B.Cu) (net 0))
 (segment (start 70.5 99) (end 71.49 99) (width 0.25) (layer B.Cu) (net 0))
 (segment (start 80.01 82.501314) (end 80.01 81.28) (width 0.25) (layer B.Cu) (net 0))
 (segment (start 80.01 87.555685) (end 80.01 82.501314) (width 0.25) (layer B.Cu) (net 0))
 (segment (start 69.815685 97.75) (end 80.01 87.555685) (width 0.25) (layer B.Cu) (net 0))
 (segment (start 69.25 97.75) (end 69.815685 97.75) (width 0.25) (layer B.Cu) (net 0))
 (segment (start 81.28 80.23) (end 81.28 88.99) (width 0.25) (layer B.Cu) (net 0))
 (segment (start 80.873599 79.603599) (end 80.873599 79.623599) (width 0.25) (layer B.Cu) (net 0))
 (segment (start 80.01 78.74) (end 80.873599 79.603599) (width 0.25) (layer B.Cu) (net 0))
 (segment (start 81.28 80.03) (end 81.28 80.23) (width 0.25) (layer B.Cu) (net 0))
 (segment (start 80.873599 79.623599) (end 81.28 80.03) (width 0.25) (layer B.Cu) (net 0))
 (segment (start 71.48 99.01) (end 81.28 89.04) (width 0.25) (layer B.Cu) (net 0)))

